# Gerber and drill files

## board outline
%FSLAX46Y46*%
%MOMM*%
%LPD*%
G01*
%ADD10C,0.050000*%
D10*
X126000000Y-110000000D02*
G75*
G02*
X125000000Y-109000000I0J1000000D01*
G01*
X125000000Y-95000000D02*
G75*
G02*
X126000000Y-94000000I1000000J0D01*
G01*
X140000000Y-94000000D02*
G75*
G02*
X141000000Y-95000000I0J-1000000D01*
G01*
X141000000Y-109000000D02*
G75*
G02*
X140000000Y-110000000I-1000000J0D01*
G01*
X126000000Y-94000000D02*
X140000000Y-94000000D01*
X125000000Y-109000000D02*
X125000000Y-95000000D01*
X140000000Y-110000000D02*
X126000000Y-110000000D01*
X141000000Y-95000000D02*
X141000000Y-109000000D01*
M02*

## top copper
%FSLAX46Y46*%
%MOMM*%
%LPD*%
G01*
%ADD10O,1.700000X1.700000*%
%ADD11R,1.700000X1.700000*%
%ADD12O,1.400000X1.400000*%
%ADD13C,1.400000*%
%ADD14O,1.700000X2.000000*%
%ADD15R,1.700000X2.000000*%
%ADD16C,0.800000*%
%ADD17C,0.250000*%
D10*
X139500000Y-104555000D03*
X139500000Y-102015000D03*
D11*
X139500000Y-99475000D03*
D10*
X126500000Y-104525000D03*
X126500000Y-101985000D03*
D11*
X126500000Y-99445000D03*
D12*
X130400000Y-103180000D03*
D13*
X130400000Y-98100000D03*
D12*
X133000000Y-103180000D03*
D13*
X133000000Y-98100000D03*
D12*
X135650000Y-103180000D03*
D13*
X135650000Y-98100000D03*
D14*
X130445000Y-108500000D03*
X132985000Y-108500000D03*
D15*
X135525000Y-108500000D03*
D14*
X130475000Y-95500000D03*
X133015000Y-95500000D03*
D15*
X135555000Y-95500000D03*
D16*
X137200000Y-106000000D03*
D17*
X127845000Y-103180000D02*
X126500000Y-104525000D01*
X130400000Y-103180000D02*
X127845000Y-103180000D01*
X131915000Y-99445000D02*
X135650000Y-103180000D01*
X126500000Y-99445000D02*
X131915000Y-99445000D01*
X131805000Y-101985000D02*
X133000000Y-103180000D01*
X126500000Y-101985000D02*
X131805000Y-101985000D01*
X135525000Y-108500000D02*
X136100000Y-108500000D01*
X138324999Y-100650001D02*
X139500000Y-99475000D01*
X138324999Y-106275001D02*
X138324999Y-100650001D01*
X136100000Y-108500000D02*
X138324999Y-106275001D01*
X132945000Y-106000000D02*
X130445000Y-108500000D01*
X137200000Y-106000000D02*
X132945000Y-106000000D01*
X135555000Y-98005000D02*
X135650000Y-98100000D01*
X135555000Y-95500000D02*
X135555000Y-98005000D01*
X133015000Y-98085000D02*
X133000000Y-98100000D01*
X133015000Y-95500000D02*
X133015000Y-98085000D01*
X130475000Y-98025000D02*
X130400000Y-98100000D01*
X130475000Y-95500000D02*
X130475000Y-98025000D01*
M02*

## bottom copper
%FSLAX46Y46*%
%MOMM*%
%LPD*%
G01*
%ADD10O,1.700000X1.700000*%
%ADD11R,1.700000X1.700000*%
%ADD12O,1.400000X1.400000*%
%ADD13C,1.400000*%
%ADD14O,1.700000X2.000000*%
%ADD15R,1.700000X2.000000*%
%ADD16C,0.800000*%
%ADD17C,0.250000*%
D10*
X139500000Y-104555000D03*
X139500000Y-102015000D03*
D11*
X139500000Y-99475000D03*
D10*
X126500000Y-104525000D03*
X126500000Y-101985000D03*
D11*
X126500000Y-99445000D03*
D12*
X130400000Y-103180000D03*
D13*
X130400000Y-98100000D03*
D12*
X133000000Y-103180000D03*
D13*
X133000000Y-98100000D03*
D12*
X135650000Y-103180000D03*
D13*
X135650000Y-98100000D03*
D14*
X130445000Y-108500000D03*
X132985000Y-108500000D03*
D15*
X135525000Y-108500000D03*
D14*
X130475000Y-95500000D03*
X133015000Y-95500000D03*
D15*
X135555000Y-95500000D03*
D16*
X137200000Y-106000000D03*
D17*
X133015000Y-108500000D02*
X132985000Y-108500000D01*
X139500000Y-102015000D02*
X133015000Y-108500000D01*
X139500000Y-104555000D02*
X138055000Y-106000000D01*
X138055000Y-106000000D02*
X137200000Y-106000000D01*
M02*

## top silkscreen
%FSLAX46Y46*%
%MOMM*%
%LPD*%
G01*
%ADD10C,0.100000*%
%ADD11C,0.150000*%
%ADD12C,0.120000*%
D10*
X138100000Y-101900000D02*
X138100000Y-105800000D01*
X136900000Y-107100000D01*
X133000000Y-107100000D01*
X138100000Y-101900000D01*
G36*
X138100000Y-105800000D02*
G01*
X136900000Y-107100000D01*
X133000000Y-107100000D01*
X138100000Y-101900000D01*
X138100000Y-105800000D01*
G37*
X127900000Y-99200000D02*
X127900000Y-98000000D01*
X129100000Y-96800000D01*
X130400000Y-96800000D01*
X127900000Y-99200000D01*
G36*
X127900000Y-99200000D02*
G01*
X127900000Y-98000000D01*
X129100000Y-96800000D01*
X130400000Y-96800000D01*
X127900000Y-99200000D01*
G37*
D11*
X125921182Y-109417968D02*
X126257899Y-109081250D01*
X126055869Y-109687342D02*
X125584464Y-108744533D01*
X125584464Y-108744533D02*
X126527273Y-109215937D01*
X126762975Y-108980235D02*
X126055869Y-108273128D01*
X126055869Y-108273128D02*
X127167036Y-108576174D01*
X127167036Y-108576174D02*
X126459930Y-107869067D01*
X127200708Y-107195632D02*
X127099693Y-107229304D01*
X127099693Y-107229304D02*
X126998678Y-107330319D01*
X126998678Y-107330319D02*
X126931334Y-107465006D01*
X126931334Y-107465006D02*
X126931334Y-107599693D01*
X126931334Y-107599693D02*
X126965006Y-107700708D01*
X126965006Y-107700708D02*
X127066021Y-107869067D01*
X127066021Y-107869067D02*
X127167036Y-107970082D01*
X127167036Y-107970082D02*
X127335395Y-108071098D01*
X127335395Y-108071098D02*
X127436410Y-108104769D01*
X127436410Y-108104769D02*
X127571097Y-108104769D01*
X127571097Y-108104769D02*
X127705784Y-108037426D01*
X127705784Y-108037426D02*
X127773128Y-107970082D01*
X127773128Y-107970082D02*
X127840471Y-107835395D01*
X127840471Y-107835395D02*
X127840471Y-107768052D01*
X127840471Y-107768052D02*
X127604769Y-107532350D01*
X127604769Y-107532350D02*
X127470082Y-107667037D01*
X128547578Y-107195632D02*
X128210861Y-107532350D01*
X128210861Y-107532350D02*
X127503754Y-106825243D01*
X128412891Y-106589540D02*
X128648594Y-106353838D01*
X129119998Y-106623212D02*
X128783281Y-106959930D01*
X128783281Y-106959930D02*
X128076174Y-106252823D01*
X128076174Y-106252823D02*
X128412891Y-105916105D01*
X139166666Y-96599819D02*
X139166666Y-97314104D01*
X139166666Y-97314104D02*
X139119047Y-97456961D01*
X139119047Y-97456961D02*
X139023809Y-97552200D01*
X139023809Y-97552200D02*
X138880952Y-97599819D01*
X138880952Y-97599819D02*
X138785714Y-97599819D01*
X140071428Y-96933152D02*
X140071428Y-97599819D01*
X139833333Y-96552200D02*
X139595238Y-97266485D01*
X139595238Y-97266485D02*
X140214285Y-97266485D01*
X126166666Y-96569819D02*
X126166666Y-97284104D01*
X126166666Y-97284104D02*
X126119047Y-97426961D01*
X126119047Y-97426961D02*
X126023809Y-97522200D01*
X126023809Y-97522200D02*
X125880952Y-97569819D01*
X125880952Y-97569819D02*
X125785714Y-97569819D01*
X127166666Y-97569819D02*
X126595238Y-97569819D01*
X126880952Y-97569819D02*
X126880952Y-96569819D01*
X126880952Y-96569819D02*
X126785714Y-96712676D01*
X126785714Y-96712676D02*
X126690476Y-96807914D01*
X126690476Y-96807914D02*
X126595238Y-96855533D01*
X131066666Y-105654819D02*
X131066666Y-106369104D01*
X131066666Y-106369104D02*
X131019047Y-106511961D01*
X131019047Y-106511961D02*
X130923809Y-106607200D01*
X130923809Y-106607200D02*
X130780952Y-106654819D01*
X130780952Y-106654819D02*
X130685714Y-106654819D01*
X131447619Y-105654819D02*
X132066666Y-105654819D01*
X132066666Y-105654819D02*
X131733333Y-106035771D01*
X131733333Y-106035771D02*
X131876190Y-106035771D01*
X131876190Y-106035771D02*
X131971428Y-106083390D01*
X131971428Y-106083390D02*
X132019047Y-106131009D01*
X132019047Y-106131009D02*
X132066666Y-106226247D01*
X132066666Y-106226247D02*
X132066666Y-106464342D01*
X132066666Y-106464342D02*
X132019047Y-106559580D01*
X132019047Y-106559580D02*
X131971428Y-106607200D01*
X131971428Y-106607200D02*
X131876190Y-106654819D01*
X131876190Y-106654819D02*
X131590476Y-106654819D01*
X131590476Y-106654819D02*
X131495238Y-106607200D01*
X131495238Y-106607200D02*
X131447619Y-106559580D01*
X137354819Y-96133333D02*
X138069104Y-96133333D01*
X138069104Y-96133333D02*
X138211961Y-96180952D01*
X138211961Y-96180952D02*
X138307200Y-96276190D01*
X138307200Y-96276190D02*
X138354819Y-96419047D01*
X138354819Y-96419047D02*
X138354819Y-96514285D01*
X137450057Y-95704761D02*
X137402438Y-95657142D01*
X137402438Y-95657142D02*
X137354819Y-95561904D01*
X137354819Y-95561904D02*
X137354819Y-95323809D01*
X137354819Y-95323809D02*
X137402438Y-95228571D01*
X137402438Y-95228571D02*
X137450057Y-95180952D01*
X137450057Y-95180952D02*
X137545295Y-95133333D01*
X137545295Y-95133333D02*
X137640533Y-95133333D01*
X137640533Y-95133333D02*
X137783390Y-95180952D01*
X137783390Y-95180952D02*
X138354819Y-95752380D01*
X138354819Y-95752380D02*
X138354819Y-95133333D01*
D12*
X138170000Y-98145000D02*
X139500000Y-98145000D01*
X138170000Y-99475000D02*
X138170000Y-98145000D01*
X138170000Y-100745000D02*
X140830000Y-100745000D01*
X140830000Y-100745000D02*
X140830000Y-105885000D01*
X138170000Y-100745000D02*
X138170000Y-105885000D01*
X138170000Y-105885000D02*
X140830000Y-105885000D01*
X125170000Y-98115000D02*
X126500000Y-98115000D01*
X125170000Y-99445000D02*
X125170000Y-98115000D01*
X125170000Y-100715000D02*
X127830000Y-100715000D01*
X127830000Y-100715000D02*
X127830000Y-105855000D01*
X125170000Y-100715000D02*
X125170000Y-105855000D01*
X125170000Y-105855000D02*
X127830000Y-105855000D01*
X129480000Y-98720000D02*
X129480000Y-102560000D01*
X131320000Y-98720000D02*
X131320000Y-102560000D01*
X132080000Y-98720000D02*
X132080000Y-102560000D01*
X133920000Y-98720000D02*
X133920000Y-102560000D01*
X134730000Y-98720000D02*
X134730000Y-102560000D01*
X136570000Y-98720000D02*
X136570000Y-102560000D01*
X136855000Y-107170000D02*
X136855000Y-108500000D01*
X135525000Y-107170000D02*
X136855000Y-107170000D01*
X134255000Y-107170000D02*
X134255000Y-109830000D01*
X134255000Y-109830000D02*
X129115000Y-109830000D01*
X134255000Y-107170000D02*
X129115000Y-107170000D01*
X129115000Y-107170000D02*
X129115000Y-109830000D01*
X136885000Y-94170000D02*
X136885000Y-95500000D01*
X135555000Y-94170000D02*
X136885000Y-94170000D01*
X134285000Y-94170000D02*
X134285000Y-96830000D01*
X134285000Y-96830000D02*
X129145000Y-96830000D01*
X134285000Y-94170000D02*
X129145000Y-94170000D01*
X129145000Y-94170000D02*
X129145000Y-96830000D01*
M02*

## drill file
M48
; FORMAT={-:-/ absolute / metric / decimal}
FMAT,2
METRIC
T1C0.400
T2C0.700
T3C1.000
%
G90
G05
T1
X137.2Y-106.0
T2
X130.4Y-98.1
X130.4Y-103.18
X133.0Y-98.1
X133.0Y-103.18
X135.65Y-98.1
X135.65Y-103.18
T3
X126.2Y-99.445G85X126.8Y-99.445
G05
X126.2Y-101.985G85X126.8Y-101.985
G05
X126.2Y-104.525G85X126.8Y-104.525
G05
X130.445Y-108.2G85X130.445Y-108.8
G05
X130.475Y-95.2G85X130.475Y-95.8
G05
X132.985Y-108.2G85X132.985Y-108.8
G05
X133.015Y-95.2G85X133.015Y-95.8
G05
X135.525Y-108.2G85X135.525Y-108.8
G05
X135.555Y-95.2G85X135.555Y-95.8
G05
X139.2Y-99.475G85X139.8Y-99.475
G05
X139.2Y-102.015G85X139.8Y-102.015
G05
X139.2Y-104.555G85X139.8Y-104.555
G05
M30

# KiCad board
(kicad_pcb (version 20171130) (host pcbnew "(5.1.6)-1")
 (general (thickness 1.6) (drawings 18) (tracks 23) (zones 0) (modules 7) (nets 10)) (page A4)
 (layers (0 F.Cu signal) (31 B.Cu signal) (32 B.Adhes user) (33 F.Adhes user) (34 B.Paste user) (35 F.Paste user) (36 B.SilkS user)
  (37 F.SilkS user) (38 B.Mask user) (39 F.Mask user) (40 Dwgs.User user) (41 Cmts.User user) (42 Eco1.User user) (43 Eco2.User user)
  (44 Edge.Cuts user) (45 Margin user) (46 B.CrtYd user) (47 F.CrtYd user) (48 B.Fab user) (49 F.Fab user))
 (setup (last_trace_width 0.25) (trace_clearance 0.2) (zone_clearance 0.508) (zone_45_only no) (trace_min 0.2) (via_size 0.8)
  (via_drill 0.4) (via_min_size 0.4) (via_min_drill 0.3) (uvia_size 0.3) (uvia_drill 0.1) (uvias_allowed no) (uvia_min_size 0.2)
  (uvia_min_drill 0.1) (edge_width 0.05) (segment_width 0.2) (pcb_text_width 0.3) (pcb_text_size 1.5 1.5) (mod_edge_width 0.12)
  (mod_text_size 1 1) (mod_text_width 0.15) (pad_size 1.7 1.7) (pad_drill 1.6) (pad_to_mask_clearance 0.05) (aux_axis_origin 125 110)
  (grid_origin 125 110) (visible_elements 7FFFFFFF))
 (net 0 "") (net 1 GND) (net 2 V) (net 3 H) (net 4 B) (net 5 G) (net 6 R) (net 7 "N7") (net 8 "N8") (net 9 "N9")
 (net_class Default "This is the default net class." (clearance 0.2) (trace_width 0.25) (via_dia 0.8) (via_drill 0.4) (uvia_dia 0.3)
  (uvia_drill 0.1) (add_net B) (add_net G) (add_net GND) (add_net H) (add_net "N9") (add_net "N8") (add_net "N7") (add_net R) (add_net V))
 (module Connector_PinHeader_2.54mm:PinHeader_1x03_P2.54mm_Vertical (layer F.Cu) (at 139.5 99.475)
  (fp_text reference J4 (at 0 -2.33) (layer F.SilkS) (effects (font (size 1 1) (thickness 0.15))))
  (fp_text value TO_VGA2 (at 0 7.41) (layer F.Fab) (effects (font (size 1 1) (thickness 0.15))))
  (fp_line (start -1.33 -1.33) (end 0 -1.33) (layer F.SilkS) (width 0.12))
  (fp_line (start -1.33 0) (end -1.33 -1.33) (layer F.SilkS) (width 0.12))
  (fp_line (start -1.33 1.27) (end 1.33 1.27) (layer F.SilkS) (width 0.12))
  (fp_line (start 1.33 1.27) (end 1.33 6.41) (layer F.SilkS) (width 0.12))
  (fp_line (start -1.33 1.27) (end -1.33 6.41) (layer F.SilkS) (width 0.12))
  (fp_line (start -1.33 6.41) (end 1.33 6.41) (layer F.SilkS) (width 0.12))
  (pad 3 thru_hole oval (at 0 5.08) (size 1.7 1.7) (drill oval 1.6 1) (layers *.Cu *.Mask) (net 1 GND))
  (pad 2 thru_hole oval (at 0 2.54) (size 1.7 1.7) (drill oval 1.6 1) (layers *.Cu *.Mask) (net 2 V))
  (pad 1 thru_hole rect (at 0 0) (size 1.7 1.7) (drill oval 1.6 1) (layers *.Cu *.Mask) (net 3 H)))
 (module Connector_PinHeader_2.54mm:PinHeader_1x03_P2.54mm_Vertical (layer F.Cu) (at 126.5 99.445)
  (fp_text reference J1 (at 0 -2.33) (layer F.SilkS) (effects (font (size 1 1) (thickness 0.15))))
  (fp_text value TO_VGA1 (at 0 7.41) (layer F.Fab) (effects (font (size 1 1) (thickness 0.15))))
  (fp_line (start -1.33 -1.33) (end 0 -1.33) (layer F.SilkS) (width 0.12))
  (fp_line (start -1.33 0) (end -1.33 -1.33) (layer F.SilkS) (width 0.12))
  (fp_line (start -1.33 1.27) (end 1.33 1.27) (layer F.SilkS) (width 0.12))
  (fp_line (start 1.33 1.27) (end 1.33 6.41) (layer F.SilkS) (width 0.12))
  (fp_line (start -1.33 1.27) (end -1.33 6.41) (layer F.SilkS) (width 0.12))
  (fp_line (start -1.33 6.41) (end 1.33 6.41) (layer F.SilkS) (width 0.12))
  (pad 3 thru_hole oval (at 0 5.08) (size 1.7 1.7) (drill oval 1.6 1) (layers *.Cu *.Mask) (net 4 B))
  (pad 2 thru_hole oval (at 0 2.54) (size 1.7 1.7) (drill oval 1.6 1) (layers *.Cu *.Mask) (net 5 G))
  (pad 1 thru_hole rect (at 0 0) (size 1.7 1.7) (drill oval 1.6 1) (layers *.Cu *.Mask) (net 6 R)))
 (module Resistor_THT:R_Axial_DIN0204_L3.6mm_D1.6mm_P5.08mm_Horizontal (layer F.Cu) (at 130.4 98.1 270)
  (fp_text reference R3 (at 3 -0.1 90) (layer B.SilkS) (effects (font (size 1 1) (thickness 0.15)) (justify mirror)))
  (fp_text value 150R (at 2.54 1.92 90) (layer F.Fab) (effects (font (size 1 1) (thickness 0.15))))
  (fp_line (start 0.62 0.92) (end 4.46 0.92) (layer F.SilkS) (width 0.12))
  (fp_line (start 0.62 -0.92) (end 4.46 -0.92) (layer F.SilkS) (width 0.12))
  (pad 2 thru_hole oval (at 5.08 0 270) (size 1.4 1.4) (drill 0.7) (layers *.Cu *.Mask) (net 4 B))
  (pad 1 thru_hole circle (at 0 0 270) (size 1.4 1.4) (drill 0.7) (layers *.Cu *.Mask) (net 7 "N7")))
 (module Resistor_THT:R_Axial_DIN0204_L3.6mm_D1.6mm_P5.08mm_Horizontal (layer F.Cu) (at 133 98.1 270)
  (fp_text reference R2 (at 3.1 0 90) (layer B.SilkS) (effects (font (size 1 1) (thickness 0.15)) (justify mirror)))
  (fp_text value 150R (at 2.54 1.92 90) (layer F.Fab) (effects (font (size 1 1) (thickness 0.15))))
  (fp_line (start 0.62 0.92) (end 4.46 0.92) (layer F.SilkS) (width 0.12))
  (fp_line (start 0.62 -0.92) (end 4.46 -0.92) (layer F.SilkS) (width 0.12))
  (pad 2 thru_hole oval (at 5.08 0 270) (size 1.4 1.4) (drill 0.7) (layers *.Cu *.Mask) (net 5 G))
  (pad 1 thru_hole circle (at 0 0 270) (size 1.4 1.4) (drill 0.7) (layers *.Cu *.Mask) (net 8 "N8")))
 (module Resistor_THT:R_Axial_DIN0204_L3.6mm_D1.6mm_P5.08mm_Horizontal (layer F.Cu) (at 135.65 98.1 270)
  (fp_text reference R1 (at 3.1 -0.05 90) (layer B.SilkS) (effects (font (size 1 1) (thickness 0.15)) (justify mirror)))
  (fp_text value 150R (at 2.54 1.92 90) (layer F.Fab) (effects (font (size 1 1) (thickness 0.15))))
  (fp_line (start 0.62 0.92) (end 4.46 0.92) (layer F.SilkS) (width 0.12))
  (fp_line (start 0.62 -0.92) (end 4.46 -0.92) (layer F.SilkS) (width 0.12))
  (pad 2 thru_hole oval (at 5.08 0 270) (size 1.4 1.4) (drill 0.7) (layers *.Cu *.Mask) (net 6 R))
  (pad 1 thru_hole circle (at 0 0 270) (size 1.4 1.4) (drill 0.7) (layers *.Cu *.Mask) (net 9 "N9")))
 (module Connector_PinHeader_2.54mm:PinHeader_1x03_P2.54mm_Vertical (layer F.Cu) (at 135.525 108.5 270)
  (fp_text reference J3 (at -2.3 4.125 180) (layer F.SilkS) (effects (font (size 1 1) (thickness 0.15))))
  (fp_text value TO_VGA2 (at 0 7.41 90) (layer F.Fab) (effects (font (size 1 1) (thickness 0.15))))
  (fp_line (start -1.33 -1.33) (end 0 -1.33) (layer F.SilkS) (width 0.12))
  (fp_line (start -1.33 0) (end -1.33 -1.33) (layer F.SilkS) (width 0.12))
  (fp_line (start -1.33 1.27) (end 1.33 1.27) (layer F.SilkS) (width 0.12))
  (fp_line (start 1.33 1.27) (end 1.33 6.41) (layer F.SilkS) (width 0.12))
  (fp_line (start -1.33 1.27) (end -1.33 6.41) (layer F.SilkS) (width 0.12))
  (fp_line (start -1.33 6.41) (end 1.33 6.41) (layer F.SilkS) (width 0.12))
  (pad 3 thru_hole oval (at 0 5.08 270) (size 2 1.7) (drill oval 1.6 1) (layers *.Cu *.Mask) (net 1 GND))
  (pad 2 thru_hole oval (at 0 2.54 270) (size 2 1.7) (drill oval 1.6 1) (layers *.Cu *.Mask) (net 2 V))
  (pad 1 thru_hole rect (at 0 0 270) (size 2 1.7) (drill oval 1.6 1) (layers *.Cu *.Mask) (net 3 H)))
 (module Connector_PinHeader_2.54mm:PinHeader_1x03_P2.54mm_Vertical (layer F.Cu) (at 135.555 95.5 270)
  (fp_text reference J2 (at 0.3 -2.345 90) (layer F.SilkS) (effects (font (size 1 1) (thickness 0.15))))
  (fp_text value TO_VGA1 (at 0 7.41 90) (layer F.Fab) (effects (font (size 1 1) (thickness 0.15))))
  (fp_line (start -1.33 -1.33) (end 0 -1.33) (layer F.SilkS) (width 0.12))
  (fp_line (start -1.33 0) (end -1.33 -1.33) (layer F.SilkS) (width 0.12))
  (fp_line (start -1.33 1.27) (end 1.33 1.27) (layer F.SilkS) (width 0.12))
  (fp_line (start 1.33 1.27) (end 1.33 6.41) (layer F.SilkS) (width 0.12))
  (fp_line (start -1.33 1.27) (end -1.33 6.41) (layer F.SilkS) (width 0.12))
  (fp_line (start -1.33 6.41) (end 1.33 6.41) (layer F.SilkS) (width 0.12))
  (pad 3 thru_hole oval (at 0 5.08 270) (size 2 1.7) (drill oval 1.6 1) (layers *.Cu *.Mask) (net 7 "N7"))
  (pad 2 thru_hole oval (at 0 2.54 270) (size 2 1.7) (drill oval 1.6 1) (layers *.Cu *.Mask) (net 8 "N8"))
  (pad 1 thru_hole rect (at 0 0 270) (size 2 1.7) (drill oval 1.6 1) (layers *.Cu *.Mask) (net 9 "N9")))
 (gr_poly (pts (xy 138.1 101.9) (xy 138.1 105.8) (xy 136.9 107.1) (xy 133 107.1)) (layer F.SilkS) (width 0.1))
 (gr_poly (pts (xy 127.9 99.2) (xy 127.9 98) (xy 129.1 96.8) (xy 130.4 96.8)) (layer F.SilkS) (width 0.1))
 (gr_arc (start 126 109) (end 125 109) (angle -90) (layer Edge.Cuts) (width 0.05))
 (gr_arc (start 126 95) (end 126 94) (angle -90) (layer Edge.Cuts) (width 0.05))
 (gr_arc (start 140 95) (end 141 95) (angle -90) (layer Edge.Cuts) (width 0.05))
 (gr_arc (start 140 109) (end 140 110) (angle -90) (layer Edge.Cuts) (width 0.05))
 (gr_line (start 126 94) (end 140 94) (layer Edge.Cuts) (width 0.05))
 (gr_line (start 125 109) (end 125 95) (layer Edge.Cuts) (width 0.05))
 (gr_line (start 140 110) (end 126 110) (layer Edge.Cuts) (width 0.05))
 (gr_line (start 141 95) (end 141 109) (layer Edge.Cuts) (width 0.05))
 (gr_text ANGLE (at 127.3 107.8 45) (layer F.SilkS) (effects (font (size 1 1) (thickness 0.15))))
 (segment (start 127.845 103.18) (end 126.5 104.525) (width 0.25) (layer F.Cu) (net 4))
 (segment (start 130.4 103.18) (end 127.845 103.18) (width 0.25) (layer F.Cu) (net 4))
 (segment (start 131.915 99.445) (end 135.65 103.18) (width 0.25) (layer F.Cu) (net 6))
 (segment (start 126.5 99.445) (end 131.915 99.445) (width 0.25) (layer F.Cu) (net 6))
 (segment (start 131.805 101.985) (end 133 103.18) (width 0.25) (layer F.Cu) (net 5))
 (segment (start 126.5 101.985) (end 131.805 101.985) (width 0.25) (layer F.Cu) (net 5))
 (segment (start 133.015 108.5) (end 132.985 108.5) (width 0.25) (layer B.Cu) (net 2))
 (segment (start 139.5 102.015) (end 133.015 108.5) (width 0.25) (layer B.Cu) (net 2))
 (segment (start 135.525 108.5) (end 136.1 108.5) (width 0.25) (layer F.Cu) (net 3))
 (segment (start 138.324999 100.650001) (end 139.5 99.475) (width 0.25) (layer F.Cu) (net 3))
 (segment (start 138.324999 106.275001) (end 138.324999 100.650001) (width 0.25) (layer F.Cu) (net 3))
 (segment (start 136.1 108.5) (end 138.324999 106.275001) (width 0.25) (layer F.Cu) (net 3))
 (segment (start 139.5 104.555) (end 138.055 106) (width 0.25) (layer B.Cu) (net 1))
 (via (at 137.2 106) (size 0.8) (drill 0.4) (layers F.Cu B.Cu) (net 1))
 (segment (start 138.055 106) (end 137.2 106) (width 0.25) (layer B.Cu) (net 1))
 (segment (start 132.945 106) (end 130.445 108.5) (width 0.25) (layer F.Cu) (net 1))
 (segment (start 137.2 106) (end 132.945 106) (width 0.25) (layer F.Cu) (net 1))
 (segment (start 135.555 98.005) (end 135.65 98.1) (width 0.25) (layer F.Cu) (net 9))
 (segment (start 135.555 95.5) (end 135.555 98.005) (width 0.25) (layer F.Cu) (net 9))
 (segment (start 133.015 98.085) (end 133 98.1) (width 0.25) (layer F.Cu) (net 8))
 (segment (start 133.015 95.5) (end 133.015 98.085) (width 0.25) (layer F.Cu) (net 8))
 (segment (start 130.475 98.025) (end 130.4 98.1) (width 0.25) (layer F.Cu) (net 7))
 (segment (start 130.475 95.5) (end 130.475 98.025) (width 0.25) (layer F.Cu) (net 7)))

